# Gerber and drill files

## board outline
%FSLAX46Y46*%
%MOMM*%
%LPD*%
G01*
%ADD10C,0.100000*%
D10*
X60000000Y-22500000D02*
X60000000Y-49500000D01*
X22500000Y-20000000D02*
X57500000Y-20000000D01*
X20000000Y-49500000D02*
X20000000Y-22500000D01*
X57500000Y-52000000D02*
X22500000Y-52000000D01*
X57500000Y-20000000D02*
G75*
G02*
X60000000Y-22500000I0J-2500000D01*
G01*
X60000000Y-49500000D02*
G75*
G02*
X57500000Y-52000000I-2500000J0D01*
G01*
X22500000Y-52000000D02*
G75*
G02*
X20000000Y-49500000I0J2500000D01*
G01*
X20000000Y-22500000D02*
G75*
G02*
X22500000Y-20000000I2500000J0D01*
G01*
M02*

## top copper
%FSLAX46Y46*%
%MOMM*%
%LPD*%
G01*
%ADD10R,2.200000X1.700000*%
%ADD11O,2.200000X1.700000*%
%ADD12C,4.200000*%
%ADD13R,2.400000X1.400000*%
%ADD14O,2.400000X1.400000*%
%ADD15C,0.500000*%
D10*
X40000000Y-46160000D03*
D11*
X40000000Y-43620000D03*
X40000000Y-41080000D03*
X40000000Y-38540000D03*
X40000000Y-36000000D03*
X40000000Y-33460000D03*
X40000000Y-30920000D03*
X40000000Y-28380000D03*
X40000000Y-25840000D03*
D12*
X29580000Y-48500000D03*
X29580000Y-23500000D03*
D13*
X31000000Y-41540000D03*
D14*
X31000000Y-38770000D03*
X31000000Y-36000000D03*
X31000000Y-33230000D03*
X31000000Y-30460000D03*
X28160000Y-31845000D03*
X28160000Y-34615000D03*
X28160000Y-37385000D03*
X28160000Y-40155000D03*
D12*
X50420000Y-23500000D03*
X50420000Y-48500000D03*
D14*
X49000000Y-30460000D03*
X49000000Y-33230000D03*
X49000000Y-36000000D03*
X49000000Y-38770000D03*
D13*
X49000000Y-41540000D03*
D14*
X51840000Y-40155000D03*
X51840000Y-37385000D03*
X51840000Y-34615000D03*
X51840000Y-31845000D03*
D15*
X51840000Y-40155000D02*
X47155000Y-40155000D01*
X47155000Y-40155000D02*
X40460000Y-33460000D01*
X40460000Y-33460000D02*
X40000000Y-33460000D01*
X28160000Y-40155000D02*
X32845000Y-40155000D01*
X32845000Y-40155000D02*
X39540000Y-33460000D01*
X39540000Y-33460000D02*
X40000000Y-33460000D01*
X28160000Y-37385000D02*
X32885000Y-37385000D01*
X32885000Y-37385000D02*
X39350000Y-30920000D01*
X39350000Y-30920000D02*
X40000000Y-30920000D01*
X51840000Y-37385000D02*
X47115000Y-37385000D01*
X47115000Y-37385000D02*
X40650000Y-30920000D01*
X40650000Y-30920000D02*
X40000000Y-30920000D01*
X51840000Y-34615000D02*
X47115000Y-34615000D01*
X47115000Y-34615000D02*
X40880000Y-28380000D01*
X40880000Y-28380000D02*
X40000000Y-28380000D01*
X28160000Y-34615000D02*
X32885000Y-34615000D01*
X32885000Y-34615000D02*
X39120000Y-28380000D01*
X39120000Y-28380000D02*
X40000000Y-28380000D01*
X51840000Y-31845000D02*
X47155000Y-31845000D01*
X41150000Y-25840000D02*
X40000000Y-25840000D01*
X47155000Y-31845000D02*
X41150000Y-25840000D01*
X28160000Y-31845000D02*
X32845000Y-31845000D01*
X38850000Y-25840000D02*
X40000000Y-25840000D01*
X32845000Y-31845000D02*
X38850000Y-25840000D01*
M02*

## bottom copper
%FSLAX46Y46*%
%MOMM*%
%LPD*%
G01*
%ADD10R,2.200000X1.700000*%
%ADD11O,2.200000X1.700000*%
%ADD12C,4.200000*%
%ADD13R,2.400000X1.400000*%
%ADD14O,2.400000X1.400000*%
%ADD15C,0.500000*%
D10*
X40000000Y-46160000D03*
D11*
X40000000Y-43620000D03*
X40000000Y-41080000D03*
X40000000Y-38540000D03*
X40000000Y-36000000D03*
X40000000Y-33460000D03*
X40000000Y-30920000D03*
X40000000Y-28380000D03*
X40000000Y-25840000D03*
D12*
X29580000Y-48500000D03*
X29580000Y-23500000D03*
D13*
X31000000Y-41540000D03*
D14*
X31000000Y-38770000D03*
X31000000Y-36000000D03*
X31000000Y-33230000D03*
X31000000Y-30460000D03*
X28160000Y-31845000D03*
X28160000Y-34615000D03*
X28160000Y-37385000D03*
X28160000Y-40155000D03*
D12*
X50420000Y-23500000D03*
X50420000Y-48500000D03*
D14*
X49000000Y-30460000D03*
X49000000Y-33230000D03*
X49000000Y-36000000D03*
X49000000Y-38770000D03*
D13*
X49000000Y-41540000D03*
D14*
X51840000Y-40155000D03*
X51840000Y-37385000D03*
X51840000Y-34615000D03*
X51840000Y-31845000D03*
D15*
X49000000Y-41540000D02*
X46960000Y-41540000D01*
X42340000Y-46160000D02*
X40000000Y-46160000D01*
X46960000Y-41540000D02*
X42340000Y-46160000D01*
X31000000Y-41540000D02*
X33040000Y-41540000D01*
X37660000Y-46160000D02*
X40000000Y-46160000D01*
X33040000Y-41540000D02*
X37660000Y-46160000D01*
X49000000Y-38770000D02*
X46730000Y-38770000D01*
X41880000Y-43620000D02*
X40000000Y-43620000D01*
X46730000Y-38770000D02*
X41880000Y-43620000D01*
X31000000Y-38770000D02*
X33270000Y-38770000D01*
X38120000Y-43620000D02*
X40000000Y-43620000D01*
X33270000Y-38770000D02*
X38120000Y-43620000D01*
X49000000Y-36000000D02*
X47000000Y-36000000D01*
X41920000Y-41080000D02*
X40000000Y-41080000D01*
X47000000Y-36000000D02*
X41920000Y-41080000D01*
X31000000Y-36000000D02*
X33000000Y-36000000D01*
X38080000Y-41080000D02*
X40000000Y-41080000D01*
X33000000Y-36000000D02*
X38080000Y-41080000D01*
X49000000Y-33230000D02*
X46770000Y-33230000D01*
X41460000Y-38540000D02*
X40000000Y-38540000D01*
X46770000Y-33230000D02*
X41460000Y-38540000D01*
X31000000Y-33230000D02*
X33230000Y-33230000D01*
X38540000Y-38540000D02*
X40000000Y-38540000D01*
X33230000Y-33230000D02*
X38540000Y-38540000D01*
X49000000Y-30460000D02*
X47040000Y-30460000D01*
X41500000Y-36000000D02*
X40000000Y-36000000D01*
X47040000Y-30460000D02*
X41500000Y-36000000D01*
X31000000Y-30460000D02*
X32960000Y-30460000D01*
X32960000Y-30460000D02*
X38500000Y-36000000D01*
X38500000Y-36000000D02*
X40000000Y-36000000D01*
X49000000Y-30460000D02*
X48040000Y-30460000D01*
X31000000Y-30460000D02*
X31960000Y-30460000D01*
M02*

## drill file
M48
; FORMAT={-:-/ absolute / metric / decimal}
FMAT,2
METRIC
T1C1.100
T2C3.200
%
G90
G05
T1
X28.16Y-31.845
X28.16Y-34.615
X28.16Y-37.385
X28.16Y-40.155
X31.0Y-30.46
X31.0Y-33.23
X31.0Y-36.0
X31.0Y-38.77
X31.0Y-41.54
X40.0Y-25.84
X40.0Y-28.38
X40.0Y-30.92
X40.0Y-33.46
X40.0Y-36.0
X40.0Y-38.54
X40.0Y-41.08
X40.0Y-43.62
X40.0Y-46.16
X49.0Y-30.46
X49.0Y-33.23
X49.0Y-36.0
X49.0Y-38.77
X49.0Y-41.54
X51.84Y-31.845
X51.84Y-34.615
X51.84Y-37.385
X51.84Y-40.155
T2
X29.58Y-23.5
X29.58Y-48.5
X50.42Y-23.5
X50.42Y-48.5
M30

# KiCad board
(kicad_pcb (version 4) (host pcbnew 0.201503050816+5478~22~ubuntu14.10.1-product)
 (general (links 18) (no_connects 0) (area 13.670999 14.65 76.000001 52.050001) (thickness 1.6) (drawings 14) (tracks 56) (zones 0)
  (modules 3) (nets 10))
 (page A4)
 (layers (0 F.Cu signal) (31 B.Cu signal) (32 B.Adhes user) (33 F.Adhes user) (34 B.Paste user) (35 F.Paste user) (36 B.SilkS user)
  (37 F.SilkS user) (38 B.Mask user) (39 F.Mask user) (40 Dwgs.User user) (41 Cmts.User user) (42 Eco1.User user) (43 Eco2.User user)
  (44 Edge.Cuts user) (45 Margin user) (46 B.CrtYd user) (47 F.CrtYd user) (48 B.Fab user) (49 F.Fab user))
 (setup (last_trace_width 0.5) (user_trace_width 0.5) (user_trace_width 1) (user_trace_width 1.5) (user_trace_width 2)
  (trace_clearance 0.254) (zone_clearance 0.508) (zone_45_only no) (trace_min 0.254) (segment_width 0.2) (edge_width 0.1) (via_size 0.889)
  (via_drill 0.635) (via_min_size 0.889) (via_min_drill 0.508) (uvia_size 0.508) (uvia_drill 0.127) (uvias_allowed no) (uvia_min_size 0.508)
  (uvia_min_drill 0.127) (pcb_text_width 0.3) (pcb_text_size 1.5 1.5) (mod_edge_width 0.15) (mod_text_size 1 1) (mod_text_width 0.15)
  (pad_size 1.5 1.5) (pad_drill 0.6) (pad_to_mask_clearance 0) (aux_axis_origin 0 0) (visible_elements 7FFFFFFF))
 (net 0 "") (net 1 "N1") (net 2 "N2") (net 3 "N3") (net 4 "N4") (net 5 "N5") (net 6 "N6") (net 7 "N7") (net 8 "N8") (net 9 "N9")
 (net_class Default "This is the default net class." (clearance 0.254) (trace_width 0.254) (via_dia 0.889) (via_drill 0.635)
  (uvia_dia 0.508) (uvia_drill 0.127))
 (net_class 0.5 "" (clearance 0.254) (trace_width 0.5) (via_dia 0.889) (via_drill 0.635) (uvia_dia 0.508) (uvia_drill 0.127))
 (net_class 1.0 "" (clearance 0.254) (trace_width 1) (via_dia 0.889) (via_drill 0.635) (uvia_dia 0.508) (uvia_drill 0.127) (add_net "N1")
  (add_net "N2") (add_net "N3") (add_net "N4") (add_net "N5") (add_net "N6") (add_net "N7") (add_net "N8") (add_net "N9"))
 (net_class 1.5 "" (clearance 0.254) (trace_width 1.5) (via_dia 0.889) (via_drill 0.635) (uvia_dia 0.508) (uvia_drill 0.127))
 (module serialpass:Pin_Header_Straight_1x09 (layer F.Cu) (at 40 36 180)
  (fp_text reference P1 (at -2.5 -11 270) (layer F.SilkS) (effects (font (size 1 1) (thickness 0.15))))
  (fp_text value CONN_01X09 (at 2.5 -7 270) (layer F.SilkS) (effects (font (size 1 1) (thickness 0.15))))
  (pad 1 thru_hole rect (at 0 -10.16 180) (size 2.2 1.7) (drill 1.1) (layers *.Cu *.Mask F.SilkS) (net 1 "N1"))
  (pad 2 thru_hole oval (at 0 -7.62 180) (size 2.2 1.7) (drill 1.1) (layers *.Cu *.Mask F.SilkS) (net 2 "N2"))
  (pad 3 thru_hole oval (at 0 -5.08 180) (size 2.2 1.7) (drill 1.1) (layers *.Cu *.Mask F.SilkS) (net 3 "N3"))
  (pad 4 thru_hole oval (at 0 -2.54 180) (size 2.2 1.7) (drill 1.1) (layers *.Cu *.Mask F.SilkS) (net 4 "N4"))
  (pad 5 thru_hole oval (at 0 0 180) (size 2.2 1.7) (drill 1.1) (layers *.Cu *.Mask F.SilkS) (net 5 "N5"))
  (pad 6 thru_hole oval (at 0 2.54 180) (size 2.2 1.7) (drill 1.1) (layers *.Cu *.Mask F.SilkS) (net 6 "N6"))
  (pad 7 thru_hole oval (at 0 5.08 180) (size 2.2 1.7) (drill 1.1) (layers *.Cu *.Mask F.SilkS) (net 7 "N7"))
  (pad 8 thru_hole oval (at 0 7.62 180) (size 2.2 1.7) (drill 1.1) (layers *.Cu *.Mask F.SilkS) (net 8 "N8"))
  (pad 9 thru_hole oval (at 0 10.16 180) (size 2.2 1.7) (drill 1.1) (layers *.Cu *.Mask F.SilkS) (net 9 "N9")))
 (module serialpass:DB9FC (layer F.Cu) (at 31 36 270)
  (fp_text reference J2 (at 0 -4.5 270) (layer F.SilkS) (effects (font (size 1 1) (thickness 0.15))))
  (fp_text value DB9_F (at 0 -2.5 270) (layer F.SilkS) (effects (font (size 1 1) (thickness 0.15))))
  (pad "" thru_hole circle (at 12.5 1.42 270) (size 4.2 4.2) (drill 3.2) (layers *.Cu *.Mask F.SilkS))
  (pad "" thru_hole circle (at -12.5 1.42 270) (size 4.2 4.2) (drill 3.2) (layers *.Cu *.Mask F.SilkS))
  (pad 1 thru_hole rect (at 5.54 0 270) (size 1.4 2.4) (drill 1.1) (layers *.Cu *.Mask F.SilkS) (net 1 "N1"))
  (pad 2 thru_hole oval (at 2.77 0 270) (size 1.4 2.4) (drill 1.1) (layers *.Cu *.Mask F.SilkS) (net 2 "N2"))
  (pad 3 thru_hole oval (at 0 0 270) (size 1.4 2.4) (drill 1.1) (layers *.Cu *.Mask F.SilkS) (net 3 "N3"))
  (pad 4 thru_hole oval (at -2.77 0 270) (size 1.4 2.4) (drill 1.1) (layers *.Cu *.Mask F.SilkS) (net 4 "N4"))
  (pad 5 thru_hole oval (at -5.54 0 270) (size 1.4 2.4) (drill 1.1) (layers *.Cu *.Mask F.SilkS) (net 5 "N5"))
  (pad 9 thru_hole oval (at -4.155 2.84 270) (size 1.4 2.4) (drill 1.1) (layers *.Cu *.Mask F.SilkS) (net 9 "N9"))
  (pad 8 thru_hole oval (at -1.385 2.84 270) (size 1.4 2.4) (drill 1.1) (layers *.Cu *.Mask F.SilkS) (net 8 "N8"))
  (pad 7 thru_hole oval (at 1.385 2.84 270) (size 1.4 2.4) (drill 1.1) (layers *.Cu *.Mask F.SilkS) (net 7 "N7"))
  (pad 6 thru_hole oval (at 4.155 2.84 270) (size 1.4 2.4) (drill 1.1) (layers *.Cu *.Mask F.SilkS) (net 6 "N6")))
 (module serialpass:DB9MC (layer F.Cu) (at 49 36 90)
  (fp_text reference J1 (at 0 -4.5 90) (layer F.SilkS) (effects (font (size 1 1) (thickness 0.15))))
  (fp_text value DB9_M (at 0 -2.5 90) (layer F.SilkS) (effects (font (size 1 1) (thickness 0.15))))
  (pad "" thru_hole circle (at 12.5 1.42 90) (size 4.2 4.2) (drill 3.2) (layers *.Cu *.Mask F.SilkS))
  (pad "" thru_hole circle (at -12.5 1.42 90) (size 4.2 4.2) (drill 3.2) (layers *.Cu *.Mask F.SilkS))
  (pad 5 thru_hole oval (at 5.54 0 90) (size 1.4 2.4) (drill 1.1) (layers *.Cu *.Mask F.SilkS) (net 5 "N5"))
  (pad 4 thru_hole oval (at 2.77 0 90) (size 1.4 2.4) (drill 1.1) (layers *.Cu *.Mask F.SilkS) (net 4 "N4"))
  (pad 3 thru_hole oval (at 0 0 90) (size 1.4 2.4) (drill 1.1) (layers *.Cu *.Mask F.SilkS) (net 3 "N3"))
  (pad 2 thru_hole oval (at -2.77 0 90) (size 1.4 2.4) (drill 1.1) (layers *.Cu *.Mask F.SilkS) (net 2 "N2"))
  (pad 1 thru_hole rect (at -5.54 0 90) (size 1.4 2.4) (drill 1.1) (layers *.Cu *.Mask F.SilkS) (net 1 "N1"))
  (pad 6 thru_hole oval (at -4.155 2.84 90) (size 1.4 2.4) (drill 1.1) (layers *.Cu *.Mask F.SilkS) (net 6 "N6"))
  (pad 7 thru_hole oval (at -1.385 2.84 90) (size 1.4 2.4) (drill 1.1) (layers *.Cu *.Mask F.SilkS) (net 7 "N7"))
  (pad 8 thru_hole oval (at 1.385 2.84 90) (size 1.4 2.4) (drill 1.1) (layers *.Cu *.Mask F.SilkS) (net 8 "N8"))
  (pad 9 thru_hole oval (at 4.155 2.84 90) (size 1.4 2.4) (drill 1.1) (layers *.Cu *.Mask F.SilkS) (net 9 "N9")))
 (gr_line (start 60 22.5) (end 60 49.5) (angle 90) (layer Edge.Cuts) (width 0.1))
 (gr_line (start 22.5 20) (end 57.5 20) (angle 90) (layer Edge.Cuts) (width 0.1))
 (gr_line (start 20 49.5) (end 20 22.5) (angle 90) (layer Edge.Cuts) (width 0.1))
 (gr_line (start 57.5 52) (end 22.5 52) (angle 90) (layer Edge.Cuts) (width 0.1))
 (gr_arc (start 57.5 22.5) (end 57.5 20) (angle 90) (layer Edge.Cuts) (width 0.1))
 (gr_arc (start 57.5 49.5) (end 60 49.5) (angle 90) (layer Edge.Cuts) (width 0.1))
 (gr_arc (start 22.5 49.5) (end 22.5 52) (angle 90) (layer Edge.Cuts) (width 0.1))
 (gr_arc (start 22.5 22.5) (end 20 22.5) (angle 90) (layer Edge.Cuts) (width 0.1))
 (segment (start 49 41.54) (end 46.96 41.54) (width 0.5) (layer B.Cu) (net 1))
 (segment (start 42.34 46.16) (end 40 46.16) (width 0.5) (layer B.Cu) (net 1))
 (segment (start 46.96 41.54) (end 42.34 46.16) (width 0.5) (layer B.Cu) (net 1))
 (segment (start 31 41.54) (end 33.04 41.54) (width 0.5) (layer B.Cu) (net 1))
 (segment (start 37.66 46.16) (end 40 46.16) (width 0.5) (layer B.Cu) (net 1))
 (segment (start 33.04 41.54) (end 37.66 46.16) (width 0.5) (layer B.Cu) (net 1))
 (segment (start 49 38.77) (end 46.73 38.77) (width 0.5) (layer B.Cu) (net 2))
 (segment (start 41.88 43.62) (end 40 43.62) (width 0.5) (layer B.Cu) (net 2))
 (segment (start 46.73 38.77) (end 41.88 43.62) (width 0.5) (layer B.Cu) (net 2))
 (segment (start 31 38.77) (end 33.27 38.77) (width 0.5) (layer B.Cu) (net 2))
 (segment (start 38.12 43.62) (end 40 43.62) (width 0.5) (layer B.Cu) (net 2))
 (segment (start 33.27 38.77) (end 38.12 43.62) (width 0.5) (layer B.Cu) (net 2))
 (segment (start 49 36) (end 47 36) (width 0.5) (layer B.Cu) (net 3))
 (segment (start 41.92 41.08) (end 40 41.08) (width 0.5) (layer B.Cu) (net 3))
 (segment (start 47 36) (end 41.92 41.08) (width 0.5) (layer B.Cu) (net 3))
 (segment (start 31 36) (end 33 36) (width 0.5) (layer B.Cu) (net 3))
 (segment (start 38.08 41.08) (end 40 41.08) (width 0.5) (layer B.Cu) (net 3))
 (segment (start 33 36) (end 38.08 41.08) (width 0.5) (layer B.Cu) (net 3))
 (segment (start 49 33.23) (end 46.77 33.23) (width 0.5) (layer B.Cu) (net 4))
 (segment (start 41.46 38.54) (end 40 38.54) (width 0.5) (layer B.Cu) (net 4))
 (segment (start 46.77 33.23) (end 41.46 38.54) (width 0.5) (layer B.Cu) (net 4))
 (segment (start 31 33.23) (end 33.23 33.23) (width 0.5) (layer B.Cu) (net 4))
 (segment (start 38.54 38.54) (end 40 38.54) (width 0.5) (layer B.Cu) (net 4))
 (segment (start 33.23 33.23) (end 38.54 38.54) (width 0.5) (layer B.Cu) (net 4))
 (segment (start 49 30.46) (end 47.04 30.46) (width 0.5) (layer B.Cu) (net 5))
 (segment (start 41.5 36) (end 40 36) (width 0.5) (layer B.Cu) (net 5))
 (segment (start 47.04 30.46) (end 41.5 36) (width 0.5) (layer B.Cu) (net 5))
 (segment (start 31 30.46) (end 32.96 30.46) (width 0.5) (layer B.Cu) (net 5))
 (segment (start 32.96 30.46) (end 38.5 36) (width 0.5) (layer B.Cu) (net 5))
 (segment (start 38.5 36) (end 40 36) (width 0.5) (layer B.Cu) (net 5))
 (segment (start 49 30.46) (end 48.04 30.46) (width 0.5) (layer B.Cu) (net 5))
 (segment (start 31 30.46) (end 31.96 30.46) (width 0.5) (layer B.Cu) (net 5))
 (segment (start 51.84 40.155) (end 47.155 40.155) (width 0.5) (layer F.Cu) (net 6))
 (segment (start 47.155 40.155) (end 40.46 33.46) (width 0.5) (layer F.Cu) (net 6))
 (segment (start 40.46 33.46) (end 40 33.46) (width 0.5) (layer F.Cu) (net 6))
 (segment (start 28.16 40.155) (end 32.845 40.155) (width 0.5) (layer F.Cu) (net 6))
 (segment (start 32.845 40.155) (end 39.54 33.46) (width 0.5) (layer F.Cu) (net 6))
 (segment (start 39.54 33.46) (end 40 33.46) (width 0.5) (layer F.Cu) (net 6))
 (segment (start 28.16 37.385) (end 32.885 37.385) (width 0.5) (layer F.Cu) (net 7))
 (segment (start 32.885 37.385) (end 39.35 30.92) (width 0.5) (layer F.Cu) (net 7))
 (segment (start 39.35 30.92) (end 40 30.92) (width 0.5) (layer F.Cu) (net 7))
 (segment (start 51.84 37.385) (end 47.115 37.385) (width 0.5) (layer F.Cu) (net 7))
 (segment (start 47.115 37.385) (end 40.65 30.92) (width 0.5) (layer F.Cu) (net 7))
 (segment (start 40.65 30.92) (end 40 30.92) (width 0.5) (layer F.Cu) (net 7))
 (segment (start 51.84 34.615) (end 47.115 34.615) (width 0.5) (layer F.Cu) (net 8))
 (segment (start 47.115 34.615) (end 40.88 28.38) (width 0.5) (layer F.Cu) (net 8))
 (segment (start 40.88 28.38) (end 40 28.38) (width 0.5) (layer F.Cu) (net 8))
 (segment (start 28.16 34.615) (end 32.885 34.615) (width 0.5) (layer F.Cu) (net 8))
 (segment (start 32.885 34.615) (end 39.12 28.38) (width 0.5) (layer F.Cu) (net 8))
 (segment (start 39.12 28.38) (end 40 28.38) (width 0.5) (layer F.Cu) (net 8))
 (segment (start 51.84 31.845) (end 47.155 31.845) (width 0.5) (layer F.Cu) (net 9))
 (segment (start 41.15 25.84) (end 40 25.84) (width 0.5) (layer F.Cu) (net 9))
 (segment (start 47.155 31.845) (end 41.15 25.84) (width 0.5) (layer F.Cu) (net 9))
 (segment (start 28.16 31.845) (end 32.845 31.845) (width 0.5) (layer F.Cu) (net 9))
 (segment (start 38.85 25.84) (end 40 25.84) (width 0.5) (layer F.Cu) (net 9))
 (segment (start 32.845 31.845) (end 38.85 25.84) (width 0.5) (layer F.Cu) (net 9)))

